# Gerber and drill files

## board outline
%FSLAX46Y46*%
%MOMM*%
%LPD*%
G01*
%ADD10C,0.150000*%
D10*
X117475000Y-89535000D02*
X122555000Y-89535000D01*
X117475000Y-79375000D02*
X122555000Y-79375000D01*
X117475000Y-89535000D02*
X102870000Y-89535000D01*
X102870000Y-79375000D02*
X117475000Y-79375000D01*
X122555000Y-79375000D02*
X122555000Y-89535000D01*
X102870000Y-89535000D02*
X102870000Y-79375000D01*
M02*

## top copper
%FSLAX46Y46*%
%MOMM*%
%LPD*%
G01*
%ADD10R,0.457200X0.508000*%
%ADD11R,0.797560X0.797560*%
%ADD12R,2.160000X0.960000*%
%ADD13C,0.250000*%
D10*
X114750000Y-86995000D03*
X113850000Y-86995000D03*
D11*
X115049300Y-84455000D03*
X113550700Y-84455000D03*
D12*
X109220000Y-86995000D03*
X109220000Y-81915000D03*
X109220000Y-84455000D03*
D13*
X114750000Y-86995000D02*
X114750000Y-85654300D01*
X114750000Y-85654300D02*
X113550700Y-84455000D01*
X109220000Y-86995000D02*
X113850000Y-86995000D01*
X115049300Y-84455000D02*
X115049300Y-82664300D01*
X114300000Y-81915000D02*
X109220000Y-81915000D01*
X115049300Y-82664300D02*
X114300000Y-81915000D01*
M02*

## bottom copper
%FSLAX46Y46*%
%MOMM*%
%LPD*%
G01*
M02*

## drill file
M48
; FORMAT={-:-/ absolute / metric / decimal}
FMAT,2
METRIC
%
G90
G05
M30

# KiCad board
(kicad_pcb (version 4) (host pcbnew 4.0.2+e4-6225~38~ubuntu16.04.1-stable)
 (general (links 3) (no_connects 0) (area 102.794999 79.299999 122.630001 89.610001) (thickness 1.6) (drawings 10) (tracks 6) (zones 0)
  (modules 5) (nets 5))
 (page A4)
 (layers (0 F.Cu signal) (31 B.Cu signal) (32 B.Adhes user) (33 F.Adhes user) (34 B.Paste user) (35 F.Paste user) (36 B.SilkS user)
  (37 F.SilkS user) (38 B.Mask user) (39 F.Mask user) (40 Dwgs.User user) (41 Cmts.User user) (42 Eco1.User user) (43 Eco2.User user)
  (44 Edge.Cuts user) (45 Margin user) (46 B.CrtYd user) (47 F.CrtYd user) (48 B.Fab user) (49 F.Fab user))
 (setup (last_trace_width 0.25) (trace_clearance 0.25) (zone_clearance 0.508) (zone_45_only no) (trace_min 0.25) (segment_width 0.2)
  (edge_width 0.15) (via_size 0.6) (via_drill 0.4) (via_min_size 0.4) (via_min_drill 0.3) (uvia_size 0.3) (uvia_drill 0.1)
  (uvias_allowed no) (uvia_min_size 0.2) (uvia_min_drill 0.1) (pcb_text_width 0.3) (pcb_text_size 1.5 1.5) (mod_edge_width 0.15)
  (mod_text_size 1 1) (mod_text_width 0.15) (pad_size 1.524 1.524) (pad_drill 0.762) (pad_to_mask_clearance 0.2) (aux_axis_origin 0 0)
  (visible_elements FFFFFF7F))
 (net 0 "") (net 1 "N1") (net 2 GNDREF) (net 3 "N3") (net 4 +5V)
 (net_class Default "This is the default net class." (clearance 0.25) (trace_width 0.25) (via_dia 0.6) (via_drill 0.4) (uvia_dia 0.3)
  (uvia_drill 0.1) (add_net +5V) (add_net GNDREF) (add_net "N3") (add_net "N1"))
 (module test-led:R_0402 (layer F.Cu) (at 114.3 86.995 180)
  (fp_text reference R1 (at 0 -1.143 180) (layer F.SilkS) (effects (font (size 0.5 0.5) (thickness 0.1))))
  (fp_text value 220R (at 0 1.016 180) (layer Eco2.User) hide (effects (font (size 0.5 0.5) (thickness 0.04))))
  (pad 1 smd rect (at -0.45 0 180) (size 0.4572 0.508) (layers F.Cu F.Paste F.Mask) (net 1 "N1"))
  (pad 2 smd rect (at 0.45 0 180) (size 0.4572 0.508) (layers F.Cu F.Paste F.Mask) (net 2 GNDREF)))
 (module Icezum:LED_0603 (layer F.Cu) (at 114.3 84.455)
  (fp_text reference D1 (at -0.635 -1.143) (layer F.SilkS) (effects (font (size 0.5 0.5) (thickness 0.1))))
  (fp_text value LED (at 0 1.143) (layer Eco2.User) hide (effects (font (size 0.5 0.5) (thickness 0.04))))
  (pad A smd rect (at 0.7493 0 180) (size 0.79756 0.79756) (layers F.Cu F.Paste F.Mask) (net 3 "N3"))
  (pad K smd rect (at -0.7493 0 180) (size 0.79756 0.79756) (layers F.Cu F.Paste F.Mask) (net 1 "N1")))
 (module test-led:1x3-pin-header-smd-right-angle (layer F.Cu) (at 109.22 84.455)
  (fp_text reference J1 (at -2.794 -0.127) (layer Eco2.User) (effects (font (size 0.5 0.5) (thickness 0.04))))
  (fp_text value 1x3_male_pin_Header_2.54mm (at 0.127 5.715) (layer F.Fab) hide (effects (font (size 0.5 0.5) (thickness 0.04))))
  (pad 1 smd rect (at 0 2.54) (size 2.16 0.96) (layers F.Cu F.Paste F.Mask) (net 2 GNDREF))
  (pad 3 smd rect (at 0 -2.54) (size 2.16 0.96) (layers F.Cu F.Paste F.Mask) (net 3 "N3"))
  (pad 2 smd rect (at 0 0) (size 2.16 0.96) (layers F.Cu F.Paste F.Mask) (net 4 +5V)))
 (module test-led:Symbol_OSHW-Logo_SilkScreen (layer F.Cu) (at 118.745 83.82)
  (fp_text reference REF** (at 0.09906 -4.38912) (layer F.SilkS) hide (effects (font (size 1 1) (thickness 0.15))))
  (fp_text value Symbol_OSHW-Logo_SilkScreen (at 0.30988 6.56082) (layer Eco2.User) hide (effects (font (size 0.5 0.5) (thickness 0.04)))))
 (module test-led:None (layer F.Cu) (at 112.7125 99.610001)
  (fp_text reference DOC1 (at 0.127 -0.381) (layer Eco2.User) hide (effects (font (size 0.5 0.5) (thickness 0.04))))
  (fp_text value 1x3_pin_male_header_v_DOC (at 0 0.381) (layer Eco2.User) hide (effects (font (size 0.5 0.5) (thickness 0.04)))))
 (gr_line (start 117.475 89.535) (end 122.555 89.535) (angle 90) (layer Edge.Cuts) (width 0.15))
 (gr_line (start 117.475 79.375) (end 122.555 79.375) (angle 90) (layer Edge.Cuts) (width 0.15))
 (gr_line (start 117.475 89.535) (end 102.87 89.535) (angle 90) (layer Edge.Cuts) (width 0.15))
 (gr_line (start 102.87 79.375) (end 117.475 79.375) (angle 90) (layer Edge.Cuts) (width 0.15))
 (gr_line (start 122.555 79.375) (end 122.555 89.535) (angle 90) (layer Edge.Cuts) (width 0.15))
 (gr_line (start 102.87 89.535) (end 102.87 79.375) (angle 90) (layer Edge.Cuts) (width 0.15))
 (segment (start 114.75 86.995) (end 114.75 85.6543) (width 0.25) (layer F.Cu) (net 1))
 (segment (start 114.75 85.6543) (end 113.5507 84.455) (width 0.25) (layer F.Cu) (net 1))
 (segment (start 109.22 86.995) (end 113.85 86.995) (width 0.25) (layer F.Cu) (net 2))
 (segment (start 115.0493 84.455) (end 115.0493 82.6643) (width 0.25) (layer F.Cu) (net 3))
 (segment (start 114.3 81.915) (end 109.22 81.915) (width 0.25) (layer F.Cu) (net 3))
 (segment (start 115.0493 82.6643) (end 114.3 81.915) (width 0.25) (layer F.Cu) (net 3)))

